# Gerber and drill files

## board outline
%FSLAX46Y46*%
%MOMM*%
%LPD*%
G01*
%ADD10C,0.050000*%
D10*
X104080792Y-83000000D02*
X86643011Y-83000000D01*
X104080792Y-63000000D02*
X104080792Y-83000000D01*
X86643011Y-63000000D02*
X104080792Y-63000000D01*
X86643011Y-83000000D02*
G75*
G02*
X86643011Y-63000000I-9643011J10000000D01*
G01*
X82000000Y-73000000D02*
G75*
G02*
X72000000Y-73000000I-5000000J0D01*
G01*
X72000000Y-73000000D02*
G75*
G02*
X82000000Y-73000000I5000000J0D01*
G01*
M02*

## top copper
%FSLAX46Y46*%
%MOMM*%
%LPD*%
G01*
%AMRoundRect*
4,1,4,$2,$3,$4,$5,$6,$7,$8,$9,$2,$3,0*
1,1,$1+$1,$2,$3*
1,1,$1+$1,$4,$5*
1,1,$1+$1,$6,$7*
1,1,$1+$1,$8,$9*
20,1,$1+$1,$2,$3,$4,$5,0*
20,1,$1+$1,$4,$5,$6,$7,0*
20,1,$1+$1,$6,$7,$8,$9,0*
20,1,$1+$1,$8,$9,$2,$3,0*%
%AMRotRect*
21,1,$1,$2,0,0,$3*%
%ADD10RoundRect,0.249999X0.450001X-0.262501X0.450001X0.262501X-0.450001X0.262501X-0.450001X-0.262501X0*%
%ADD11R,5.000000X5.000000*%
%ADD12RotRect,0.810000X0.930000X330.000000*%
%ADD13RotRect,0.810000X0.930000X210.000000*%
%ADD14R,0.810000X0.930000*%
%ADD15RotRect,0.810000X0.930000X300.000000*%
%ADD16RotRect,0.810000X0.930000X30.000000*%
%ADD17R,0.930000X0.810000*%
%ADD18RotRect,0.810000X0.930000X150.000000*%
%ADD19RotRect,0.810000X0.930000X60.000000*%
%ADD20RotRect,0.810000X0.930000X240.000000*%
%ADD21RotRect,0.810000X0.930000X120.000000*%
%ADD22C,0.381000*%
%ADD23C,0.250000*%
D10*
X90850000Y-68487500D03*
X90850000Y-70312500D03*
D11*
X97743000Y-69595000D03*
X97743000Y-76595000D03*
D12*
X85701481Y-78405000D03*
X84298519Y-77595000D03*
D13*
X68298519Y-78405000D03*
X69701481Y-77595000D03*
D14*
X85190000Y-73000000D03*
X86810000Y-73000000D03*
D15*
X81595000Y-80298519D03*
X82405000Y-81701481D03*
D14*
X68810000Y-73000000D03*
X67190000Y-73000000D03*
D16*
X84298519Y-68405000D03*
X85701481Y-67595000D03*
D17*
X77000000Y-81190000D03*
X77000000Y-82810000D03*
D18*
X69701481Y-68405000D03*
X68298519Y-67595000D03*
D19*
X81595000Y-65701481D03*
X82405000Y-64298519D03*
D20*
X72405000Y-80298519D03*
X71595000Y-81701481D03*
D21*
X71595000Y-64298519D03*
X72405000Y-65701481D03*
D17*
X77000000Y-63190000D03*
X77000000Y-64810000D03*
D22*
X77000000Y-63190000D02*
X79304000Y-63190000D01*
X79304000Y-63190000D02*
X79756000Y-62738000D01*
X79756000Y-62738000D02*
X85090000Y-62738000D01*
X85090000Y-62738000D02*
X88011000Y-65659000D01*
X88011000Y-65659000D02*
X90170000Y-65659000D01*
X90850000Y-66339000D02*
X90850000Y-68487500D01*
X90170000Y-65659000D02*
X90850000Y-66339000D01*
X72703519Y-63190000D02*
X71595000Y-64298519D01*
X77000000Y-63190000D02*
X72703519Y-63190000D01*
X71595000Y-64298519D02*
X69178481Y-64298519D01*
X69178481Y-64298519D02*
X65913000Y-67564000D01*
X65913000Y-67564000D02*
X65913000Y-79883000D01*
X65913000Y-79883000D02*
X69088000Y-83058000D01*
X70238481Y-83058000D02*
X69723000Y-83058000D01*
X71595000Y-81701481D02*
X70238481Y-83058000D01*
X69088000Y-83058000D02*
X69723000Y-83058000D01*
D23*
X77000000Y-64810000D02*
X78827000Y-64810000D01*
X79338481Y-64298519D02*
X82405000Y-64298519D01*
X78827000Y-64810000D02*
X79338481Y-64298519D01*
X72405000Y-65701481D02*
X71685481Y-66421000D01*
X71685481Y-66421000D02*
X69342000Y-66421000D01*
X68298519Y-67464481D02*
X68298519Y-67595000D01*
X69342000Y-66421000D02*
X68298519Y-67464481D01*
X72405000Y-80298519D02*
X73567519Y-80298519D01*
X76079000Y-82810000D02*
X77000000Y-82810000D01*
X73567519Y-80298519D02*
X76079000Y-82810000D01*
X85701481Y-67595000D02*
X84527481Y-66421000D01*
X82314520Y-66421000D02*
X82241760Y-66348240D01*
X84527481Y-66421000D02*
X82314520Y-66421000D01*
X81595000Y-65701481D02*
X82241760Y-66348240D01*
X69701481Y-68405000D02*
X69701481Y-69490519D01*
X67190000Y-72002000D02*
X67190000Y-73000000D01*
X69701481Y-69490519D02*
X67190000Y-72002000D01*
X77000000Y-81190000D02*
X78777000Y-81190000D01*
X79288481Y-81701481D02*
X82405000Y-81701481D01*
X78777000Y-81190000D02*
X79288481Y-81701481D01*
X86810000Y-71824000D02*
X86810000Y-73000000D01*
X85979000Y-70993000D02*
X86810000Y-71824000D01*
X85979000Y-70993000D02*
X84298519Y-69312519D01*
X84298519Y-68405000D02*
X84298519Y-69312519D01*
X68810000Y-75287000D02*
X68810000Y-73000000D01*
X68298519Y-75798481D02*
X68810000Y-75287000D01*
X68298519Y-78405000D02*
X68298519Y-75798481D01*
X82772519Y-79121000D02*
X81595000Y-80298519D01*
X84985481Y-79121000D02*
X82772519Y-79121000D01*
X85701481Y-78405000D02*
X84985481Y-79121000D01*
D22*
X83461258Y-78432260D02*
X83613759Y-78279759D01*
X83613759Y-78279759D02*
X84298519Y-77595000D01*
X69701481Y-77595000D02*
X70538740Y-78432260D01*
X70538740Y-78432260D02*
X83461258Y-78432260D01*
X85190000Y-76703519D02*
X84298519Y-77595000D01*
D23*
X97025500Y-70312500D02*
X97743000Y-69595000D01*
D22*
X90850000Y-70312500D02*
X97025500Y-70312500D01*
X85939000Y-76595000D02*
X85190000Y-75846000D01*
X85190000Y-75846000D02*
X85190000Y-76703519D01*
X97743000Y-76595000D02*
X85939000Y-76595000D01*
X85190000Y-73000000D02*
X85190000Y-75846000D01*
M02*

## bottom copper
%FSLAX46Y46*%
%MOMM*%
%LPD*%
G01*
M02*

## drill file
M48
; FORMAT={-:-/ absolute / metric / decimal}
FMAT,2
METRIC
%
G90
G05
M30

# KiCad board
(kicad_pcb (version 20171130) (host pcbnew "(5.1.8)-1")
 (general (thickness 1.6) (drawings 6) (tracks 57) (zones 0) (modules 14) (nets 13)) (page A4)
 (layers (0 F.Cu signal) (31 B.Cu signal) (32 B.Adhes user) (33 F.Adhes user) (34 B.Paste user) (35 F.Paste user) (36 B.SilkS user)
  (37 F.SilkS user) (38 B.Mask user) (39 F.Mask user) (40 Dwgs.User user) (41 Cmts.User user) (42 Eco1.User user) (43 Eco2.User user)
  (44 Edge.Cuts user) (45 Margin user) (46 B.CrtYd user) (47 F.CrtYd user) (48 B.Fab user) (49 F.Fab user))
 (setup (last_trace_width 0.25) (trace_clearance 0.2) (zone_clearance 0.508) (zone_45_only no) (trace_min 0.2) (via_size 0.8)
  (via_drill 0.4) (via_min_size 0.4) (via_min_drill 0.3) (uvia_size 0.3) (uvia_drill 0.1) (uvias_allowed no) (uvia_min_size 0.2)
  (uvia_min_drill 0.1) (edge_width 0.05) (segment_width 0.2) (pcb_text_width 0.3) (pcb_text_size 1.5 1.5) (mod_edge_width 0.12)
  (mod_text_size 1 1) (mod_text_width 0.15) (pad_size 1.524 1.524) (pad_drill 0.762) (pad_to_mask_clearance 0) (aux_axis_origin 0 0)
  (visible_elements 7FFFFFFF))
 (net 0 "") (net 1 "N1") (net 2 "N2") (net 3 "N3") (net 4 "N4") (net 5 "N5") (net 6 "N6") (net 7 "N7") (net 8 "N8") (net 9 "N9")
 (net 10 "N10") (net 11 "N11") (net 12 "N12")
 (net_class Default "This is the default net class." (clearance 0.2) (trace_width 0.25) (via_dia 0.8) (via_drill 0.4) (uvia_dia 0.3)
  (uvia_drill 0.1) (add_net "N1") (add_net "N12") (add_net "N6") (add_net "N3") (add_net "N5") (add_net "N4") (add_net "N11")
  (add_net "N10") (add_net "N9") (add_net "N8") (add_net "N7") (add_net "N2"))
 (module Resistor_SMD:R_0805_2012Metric (layer F.Cu) (at 90.85 69.4 90)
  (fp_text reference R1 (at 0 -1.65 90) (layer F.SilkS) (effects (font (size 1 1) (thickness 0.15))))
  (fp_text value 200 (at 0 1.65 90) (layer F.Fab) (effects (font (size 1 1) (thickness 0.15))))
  (pad 2 smd roundrect (at 0.9125 0 90) (size 1.025 1.4) (layers F.Cu F.Paste F.Mask) (roundrect_rratio 0.2439014634146341) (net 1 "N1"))
  (pad 1 smd roundrect (at -0.9125 0 90) (size 1.025 1.4) (layers F.Cu F.Paste F.Mask) (roundrect_rratio 0.2439014634146341) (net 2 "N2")))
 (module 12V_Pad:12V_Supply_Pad (layer F.Cu) (at 102.743 65.595 270)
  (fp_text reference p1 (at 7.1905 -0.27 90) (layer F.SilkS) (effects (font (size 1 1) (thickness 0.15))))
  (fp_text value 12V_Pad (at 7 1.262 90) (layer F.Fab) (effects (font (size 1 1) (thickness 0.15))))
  (pad 1 smd rect (at 4 5 270) (size 5 5) (layers F.Cu F.Paste F.Mask) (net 2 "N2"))
  (pad 2 smd rect (at 11 5 270) (size 5 5) (layers F.Cu F.Paste F.Mask) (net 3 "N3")))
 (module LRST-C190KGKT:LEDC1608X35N (layer F.Cu) (at 85 78 330)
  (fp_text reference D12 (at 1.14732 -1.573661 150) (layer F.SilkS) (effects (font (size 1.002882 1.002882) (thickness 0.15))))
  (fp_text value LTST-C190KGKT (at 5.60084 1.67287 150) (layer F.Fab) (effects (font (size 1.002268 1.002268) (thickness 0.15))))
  (pad A smd rect (at 0.81 0 330) (size 0.81 0.93) (layers F.Cu F.Paste F.Mask) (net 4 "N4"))
  (pad C smd rect (at -0.81 0 330) (size 0.81 0.93) (layers F.Cu F.Paste F.Mask) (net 3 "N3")))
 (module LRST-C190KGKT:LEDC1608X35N (layer F.Cu) (at 69 78 210)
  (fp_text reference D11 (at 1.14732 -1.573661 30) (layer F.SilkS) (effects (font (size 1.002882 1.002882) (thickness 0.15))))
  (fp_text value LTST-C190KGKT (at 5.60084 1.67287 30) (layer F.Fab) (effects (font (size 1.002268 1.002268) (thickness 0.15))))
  (pad A smd rect (at 0.81 0 210) (size 0.81 0.93) (layers F.Cu F.Paste F.Mask) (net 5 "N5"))
  (pad C smd rect (at -0.81 0 210) (size 0.81 0.93) (layers F.Cu F.Paste F.Mask) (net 3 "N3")))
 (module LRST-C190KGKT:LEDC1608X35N (layer F.Cu) (at 86 73)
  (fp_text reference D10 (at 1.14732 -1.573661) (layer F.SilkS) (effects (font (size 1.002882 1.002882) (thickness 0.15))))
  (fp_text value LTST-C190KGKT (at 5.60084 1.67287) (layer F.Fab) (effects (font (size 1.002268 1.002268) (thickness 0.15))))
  (pad C smd rect (at -0.81 0) (size 0.81 0.93) (layers F.Cu F.Paste F.Mask) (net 3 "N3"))
  (pad A smd rect (at 0.81 0) (size 0.81 0.93) (layers F.Cu F.Paste F.Mask) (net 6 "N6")))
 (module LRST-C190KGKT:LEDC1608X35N (layer F.Cu) (at 82 81 300)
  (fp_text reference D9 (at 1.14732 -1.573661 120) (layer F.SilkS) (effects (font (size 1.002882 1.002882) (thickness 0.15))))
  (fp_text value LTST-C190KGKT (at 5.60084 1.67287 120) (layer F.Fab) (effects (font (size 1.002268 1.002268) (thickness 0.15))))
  (pad C smd rect (at -0.81 0 300) (size 0.81 0.93) (layers F.Cu F.Paste F.Mask) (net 4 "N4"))
  (pad A smd rect (at 0.81 0 300) (size 0.81 0.93) (layers F.Cu F.Paste F.Mask) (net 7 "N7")))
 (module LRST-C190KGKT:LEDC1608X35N (layer F.Cu) (at 68 73 180)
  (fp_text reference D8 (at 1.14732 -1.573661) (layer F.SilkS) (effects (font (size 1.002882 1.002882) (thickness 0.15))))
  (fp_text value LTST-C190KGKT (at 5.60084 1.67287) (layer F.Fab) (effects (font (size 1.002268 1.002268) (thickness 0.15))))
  (pad C smd rect (at -0.81 0 180) (size 0.81 0.93) (layers F.Cu F.Paste F.Mask) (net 5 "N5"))
  (pad A smd rect (at 0.81 0 180) (size 0.81 0.93) (layers F.Cu F.Paste F.Mask) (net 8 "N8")))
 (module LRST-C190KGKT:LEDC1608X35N (layer F.Cu) (at 85 68 30)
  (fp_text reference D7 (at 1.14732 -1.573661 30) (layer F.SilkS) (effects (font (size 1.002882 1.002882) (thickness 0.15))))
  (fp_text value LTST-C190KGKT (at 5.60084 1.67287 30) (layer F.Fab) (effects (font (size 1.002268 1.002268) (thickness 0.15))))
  (pad C smd rect (at -0.81 0 30) (size 0.81 0.93) (layers F.Cu F.Paste F.Mask) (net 6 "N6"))
  (pad A smd rect (at 0.81 0 30) (size 0.81 0.93) (layers F.Cu F.Paste F.Mask) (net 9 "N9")))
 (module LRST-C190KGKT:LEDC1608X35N (layer F.Cu) (at 77 82 270)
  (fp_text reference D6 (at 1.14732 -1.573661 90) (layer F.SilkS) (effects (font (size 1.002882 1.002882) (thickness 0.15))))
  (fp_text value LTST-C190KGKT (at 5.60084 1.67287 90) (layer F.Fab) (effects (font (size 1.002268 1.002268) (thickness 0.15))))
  (pad C smd rect (at -0.81 0 270) (size 0.81 0.93) (layers F.Cu F.Paste F.Mask) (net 7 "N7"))
  (pad A smd rect (at 0.81 0 270) (size 0.81 0.93) (layers F.Cu F.Paste F.Mask) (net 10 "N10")))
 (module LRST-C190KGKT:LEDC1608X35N (layer F.Cu) (at 69 68 150)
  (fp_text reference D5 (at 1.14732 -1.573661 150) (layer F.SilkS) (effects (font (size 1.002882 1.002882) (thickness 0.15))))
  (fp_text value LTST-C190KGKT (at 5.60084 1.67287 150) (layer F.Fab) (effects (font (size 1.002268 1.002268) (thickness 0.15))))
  (pad C smd rect (at -0.81 0 150) (size 0.81 0.93) (layers F.Cu F.Paste F.Mask) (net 8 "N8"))
  (pad A smd rect (at 0.81 0 150) (size 0.81 0.93) (layers F.Cu F.Paste F.Mask) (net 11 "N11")))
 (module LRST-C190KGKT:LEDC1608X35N (layer F.Cu) (at 82 65 60)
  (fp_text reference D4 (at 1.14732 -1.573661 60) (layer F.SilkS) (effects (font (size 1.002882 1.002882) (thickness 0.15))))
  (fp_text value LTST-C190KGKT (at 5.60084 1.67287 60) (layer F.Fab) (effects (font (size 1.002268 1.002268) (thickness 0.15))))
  (pad C smd rect (at -0.81 0 60) (size 0.81 0.93) (layers F.Cu F.Paste F.Mask) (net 9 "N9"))
  (pad A smd rect (at 0.81 0 60) (size 0.81 0.93) (layers F.Cu F.Paste F.Mask) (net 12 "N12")))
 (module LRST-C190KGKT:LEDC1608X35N (layer F.Cu) (at 72 81 240)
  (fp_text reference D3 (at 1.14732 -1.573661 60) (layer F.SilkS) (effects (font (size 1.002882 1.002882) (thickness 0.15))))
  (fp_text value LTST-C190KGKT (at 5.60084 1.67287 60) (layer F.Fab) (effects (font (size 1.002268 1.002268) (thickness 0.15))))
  (pad C smd rect (at -0.81 0 240) (size 0.81 0.93) (layers F.Cu F.Paste F.Mask) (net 10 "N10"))
  (pad A smd rect (at 0.81 0 240) (size 0.81 0.93) (layers F.Cu F.Paste F.Mask) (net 1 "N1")))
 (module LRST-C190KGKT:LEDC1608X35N (layer F.Cu) (at 72 65 120)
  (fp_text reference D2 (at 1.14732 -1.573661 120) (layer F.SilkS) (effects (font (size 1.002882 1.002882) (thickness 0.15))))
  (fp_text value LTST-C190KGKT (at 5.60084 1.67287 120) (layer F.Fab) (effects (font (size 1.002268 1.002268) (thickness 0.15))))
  (pad A smd rect (at 0.81 0 120) (size 0.81 0.93) (layers F.Cu F.Paste F.Mask) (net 1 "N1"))
  (pad C smd rect (at -0.81 0 120) (size 0.81 0.93) (layers F.Cu F.Paste F.Mask) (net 11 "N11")))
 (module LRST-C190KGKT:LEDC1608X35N (layer F.Cu) (at 77 64 90)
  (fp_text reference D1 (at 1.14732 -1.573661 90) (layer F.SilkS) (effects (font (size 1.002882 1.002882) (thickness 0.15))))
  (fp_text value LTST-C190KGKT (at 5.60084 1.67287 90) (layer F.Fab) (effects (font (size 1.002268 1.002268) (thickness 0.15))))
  (pad A smd rect (at 0.81 0 90) (size 0.81 0.93) (layers F.Cu F.Paste F.Mask) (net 1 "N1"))
  (pad C smd rect (at -0.81 0 90) (size 0.81 0.93) (layers F.Cu F.Paste F.Mask) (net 12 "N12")))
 (gr_line (start 104.080792 83) (end 86.643011 83) (layer Edge.Cuts) (width 0.05))
 (gr_line (start 104.080792 63) (end 104.080792 83) (layer Edge.Cuts) (width 0.05))
 (gr_line (start 86.643011 63) (end 104.080792 63) (layer Edge.Cuts) (width 0.05))
 (gr_arc (start 77 73) (end 86.643011 63) (angle -267.9176611) (layer Edge.Cuts) (width 0.05))
 (gr_circle (center 77 73) (end 82 73) (layer Edge.Cuts) (width 0.05))
 (segment (start 77 63.19) (end 79.304 63.19) (width 0.381) (layer F.Cu) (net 1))
 (segment (start 79.304 63.19) (end 79.756 62.738) (width 0.381) (layer F.Cu) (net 1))
 (segment (start 79.756 62.738) (end 85.09 62.738) (width 0.381) (layer F.Cu) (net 1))
 (segment (start 85.09 62.738) (end 88.011 65.659) (width 0.381) (layer F.Cu) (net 1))
 (segment (start 88.011 65.659) (end 90.17 65.659) (width 0.381) (layer F.Cu) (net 1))
 (segment (start 90.85 66.339) (end 90.85 68.4875) (width 0.381) (layer F.Cu) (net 1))
 (segment (start 90.17 65.659) (end 90.85 66.339) (width 0.381) (layer F.Cu) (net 1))
 (segment (start 72.703519 63.19) (end 71.595 64.298519) (width 0.381) (layer F.Cu) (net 1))
 (segment (start 77 63.19) (end 72.703519 63.19) (width 0.381) (layer F.Cu) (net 1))
 (segment (start 71.595 64.298519) (end 69.178481 64.298519) (width 0.381) (layer F.Cu) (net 1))
 (segment (start 69.178481 64.298519) (end 65.913 67.564) (width 0.381) (layer F.Cu) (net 1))
 (segment (start 65.913 67.564) (end 65.913 79.883) (width 0.381) (layer F.Cu) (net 1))
 (segment (start 65.913 79.883) (end 69.088 83.058) (width 0.381) (layer F.Cu) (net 1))
 (segment (start 70.238481 83.058) (end 69.723 83.058) (width 0.381) (layer F.Cu) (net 1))
 (segment (start 71.595 81.701481) (end 70.238481 83.058) (width 0.381) (layer F.Cu) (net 1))
 (segment (start 69.088 83.058) (end 69.723 83.058) (width 0.381) (layer F.Cu) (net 1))
 (segment (start 77 64.81) (end 78.827 64.81) (width 0.25) (layer F.Cu) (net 12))
 (segment (start 79.338481 64.298519) (end 82.405 64.298519) (width 0.25) (layer F.Cu) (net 12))
 (segment (start 78.827 64.81) (end 79.338481 64.298519) (width 0.25) (layer F.Cu) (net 12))
 (segment (start 72.405 65.701481) (end 71.685481 66.421) (width 0.25) (layer F.Cu) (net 11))
 (segment (start 71.685481 66.421) (end 69.342 66.421) (width 0.25) (layer F.Cu) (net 11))
 (segment (start 68.298519 67.464481) (end 68.298519 67.595) (width 0.25) (layer F.Cu) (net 11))
 (segment (start 69.342 66.421) (end 68.298519 67.464481) (width 0.25) (layer F.Cu) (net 11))
 (segment (start 72.405 80.298519) (end 73.567519 80.298519) (width 0.25) (layer F.Cu) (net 10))
 (segment (start 76.079 82.81) (end 77 82.81) (width 0.25) (layer F.Cu) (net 10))
 (segment (start 73.567519 80.298519) (end 76.079 82.81) (width 0.25) (layer F.Cu) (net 10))
 (segment (start 85.701481 67.595) (end 84.527481 66.421) (width 0.25) (layer F.Cu) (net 9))
 (segment (start 82.31452 66.421) (end 82.24176 66.34824) (width 0.25) (layer F.Cu) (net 9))
 (segment (start 84.527481 66.421) (end 82.31452 66.421) (width 0.25) (layer F.Cu) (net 9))
 (segment (start 81.595 65.701481) (end 82.24176 66.34824) (width 0.25) (layer F.Cu) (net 9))
 (segment (start 69.701481 68.405) (end 69.701481 69.490519) (width 0.25) (layer F.Cu) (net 8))
 (segment (start 67.19 72.002) (end 67.19 73) (width 0.25) (layer F.Cu) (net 8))
 (segment (start 69.701481 69.490519) (end 67.19 72.002) (width 0.25) (layer F.Cu) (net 8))
 (segment (start 77 81.19) (end 78.777 81.19) (width 0.25) (layer F.Cu) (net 7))
 (segment (start 79.288481 81.701481) (end 82.405 81.701481) (width 0.25) (layer F.Cu) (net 7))
 (segment (start 78.777 81.19) (end 79.288481 81.701481) (width 0.25) (layer F.Cu) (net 7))
 (segment (start 86.81 71.824) (end 86.81 73) (width 0.25) (layer F.Cu) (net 6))
 (segment (start 85.979 70.993) (end 86.81 71.824) (width 0.25) (layer F.Cu) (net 6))
 (segment (start 85.979 70.993) (end 84.298519 69.312519) (width 0.25) (layer F.Cu) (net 6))
 (segment (start 84.298519 68.405) (end 84.298519 69.312519) (width 0.25) (layer F.Cu) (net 6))
 (segment (start 68.81 75.287) (end 68.81 73) (width 0.25) (layer F.Cu) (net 5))
 (segment (start 68.298519 75.798481) (end 68.81 75.287) (width 0.25) (layer F.Cu) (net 5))
 (segment (start 68.298519 78.405) (end 68.298519 75.798481) (width 0.25) (layer F.Cu) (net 5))
 (segment (start 82.772519 79.121) (end 81.595 80.298519) (width 0.25) (layer F.Cu) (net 4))
 (segment (start 84.985481 79.121) (end 82.772519 79.121) (width 0.25) (layer F.Cu) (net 4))
 (segment (start 85.701481 78.405) (end 84.985481 79.121) (width 0.25) (layer F.Cu) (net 4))
 (segment (start 83.461258 78.43226) (end 83.613759 78.279759) (width 0.381) (layer F.Cu) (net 3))
 (segment (start 83.613759 78.279759) (end 84.298519 77.595) (width 0.381) (layer F.Cu) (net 3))
 (segment (start 69.701481 77.595) (end 70.53874 78.43226) (width 0.381) (layer F.Cu) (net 3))
 (segment (start 70.53874 78.43226) (end 83.461258 78.43226) (width 0.381) (layer F.Cu) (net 3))
 (segment (start 85.19 76.703519) (end 84.298519 77.595) (width 0.381) (layer F.Cu) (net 3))
 (segment (start 97.0255 70.3125) (end 97.743 69.595) (width 0.25) (layer F.Cu) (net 2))
 (segment (start 90.85 70.3125) (end 97.0255 70.3125) (width 0.381) (layer F.Cu) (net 2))
 (segment (start 85.939 76.595) (end 85.19 75.846) (width 0.381) (layer F.Cu) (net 3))
 (segment (start 85.19 75.846) (end 85.19 76.703519) (width 0.381) (layer F.Cu) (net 3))
 (segment (start 97.743 76.595) (end 85.939 76.595) (width 0.381) (layer F.Cu) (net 3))
 (segment (start 85.19 73) (end 85.19 75.846) (width 0.381) (layer F.Cu) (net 3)))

